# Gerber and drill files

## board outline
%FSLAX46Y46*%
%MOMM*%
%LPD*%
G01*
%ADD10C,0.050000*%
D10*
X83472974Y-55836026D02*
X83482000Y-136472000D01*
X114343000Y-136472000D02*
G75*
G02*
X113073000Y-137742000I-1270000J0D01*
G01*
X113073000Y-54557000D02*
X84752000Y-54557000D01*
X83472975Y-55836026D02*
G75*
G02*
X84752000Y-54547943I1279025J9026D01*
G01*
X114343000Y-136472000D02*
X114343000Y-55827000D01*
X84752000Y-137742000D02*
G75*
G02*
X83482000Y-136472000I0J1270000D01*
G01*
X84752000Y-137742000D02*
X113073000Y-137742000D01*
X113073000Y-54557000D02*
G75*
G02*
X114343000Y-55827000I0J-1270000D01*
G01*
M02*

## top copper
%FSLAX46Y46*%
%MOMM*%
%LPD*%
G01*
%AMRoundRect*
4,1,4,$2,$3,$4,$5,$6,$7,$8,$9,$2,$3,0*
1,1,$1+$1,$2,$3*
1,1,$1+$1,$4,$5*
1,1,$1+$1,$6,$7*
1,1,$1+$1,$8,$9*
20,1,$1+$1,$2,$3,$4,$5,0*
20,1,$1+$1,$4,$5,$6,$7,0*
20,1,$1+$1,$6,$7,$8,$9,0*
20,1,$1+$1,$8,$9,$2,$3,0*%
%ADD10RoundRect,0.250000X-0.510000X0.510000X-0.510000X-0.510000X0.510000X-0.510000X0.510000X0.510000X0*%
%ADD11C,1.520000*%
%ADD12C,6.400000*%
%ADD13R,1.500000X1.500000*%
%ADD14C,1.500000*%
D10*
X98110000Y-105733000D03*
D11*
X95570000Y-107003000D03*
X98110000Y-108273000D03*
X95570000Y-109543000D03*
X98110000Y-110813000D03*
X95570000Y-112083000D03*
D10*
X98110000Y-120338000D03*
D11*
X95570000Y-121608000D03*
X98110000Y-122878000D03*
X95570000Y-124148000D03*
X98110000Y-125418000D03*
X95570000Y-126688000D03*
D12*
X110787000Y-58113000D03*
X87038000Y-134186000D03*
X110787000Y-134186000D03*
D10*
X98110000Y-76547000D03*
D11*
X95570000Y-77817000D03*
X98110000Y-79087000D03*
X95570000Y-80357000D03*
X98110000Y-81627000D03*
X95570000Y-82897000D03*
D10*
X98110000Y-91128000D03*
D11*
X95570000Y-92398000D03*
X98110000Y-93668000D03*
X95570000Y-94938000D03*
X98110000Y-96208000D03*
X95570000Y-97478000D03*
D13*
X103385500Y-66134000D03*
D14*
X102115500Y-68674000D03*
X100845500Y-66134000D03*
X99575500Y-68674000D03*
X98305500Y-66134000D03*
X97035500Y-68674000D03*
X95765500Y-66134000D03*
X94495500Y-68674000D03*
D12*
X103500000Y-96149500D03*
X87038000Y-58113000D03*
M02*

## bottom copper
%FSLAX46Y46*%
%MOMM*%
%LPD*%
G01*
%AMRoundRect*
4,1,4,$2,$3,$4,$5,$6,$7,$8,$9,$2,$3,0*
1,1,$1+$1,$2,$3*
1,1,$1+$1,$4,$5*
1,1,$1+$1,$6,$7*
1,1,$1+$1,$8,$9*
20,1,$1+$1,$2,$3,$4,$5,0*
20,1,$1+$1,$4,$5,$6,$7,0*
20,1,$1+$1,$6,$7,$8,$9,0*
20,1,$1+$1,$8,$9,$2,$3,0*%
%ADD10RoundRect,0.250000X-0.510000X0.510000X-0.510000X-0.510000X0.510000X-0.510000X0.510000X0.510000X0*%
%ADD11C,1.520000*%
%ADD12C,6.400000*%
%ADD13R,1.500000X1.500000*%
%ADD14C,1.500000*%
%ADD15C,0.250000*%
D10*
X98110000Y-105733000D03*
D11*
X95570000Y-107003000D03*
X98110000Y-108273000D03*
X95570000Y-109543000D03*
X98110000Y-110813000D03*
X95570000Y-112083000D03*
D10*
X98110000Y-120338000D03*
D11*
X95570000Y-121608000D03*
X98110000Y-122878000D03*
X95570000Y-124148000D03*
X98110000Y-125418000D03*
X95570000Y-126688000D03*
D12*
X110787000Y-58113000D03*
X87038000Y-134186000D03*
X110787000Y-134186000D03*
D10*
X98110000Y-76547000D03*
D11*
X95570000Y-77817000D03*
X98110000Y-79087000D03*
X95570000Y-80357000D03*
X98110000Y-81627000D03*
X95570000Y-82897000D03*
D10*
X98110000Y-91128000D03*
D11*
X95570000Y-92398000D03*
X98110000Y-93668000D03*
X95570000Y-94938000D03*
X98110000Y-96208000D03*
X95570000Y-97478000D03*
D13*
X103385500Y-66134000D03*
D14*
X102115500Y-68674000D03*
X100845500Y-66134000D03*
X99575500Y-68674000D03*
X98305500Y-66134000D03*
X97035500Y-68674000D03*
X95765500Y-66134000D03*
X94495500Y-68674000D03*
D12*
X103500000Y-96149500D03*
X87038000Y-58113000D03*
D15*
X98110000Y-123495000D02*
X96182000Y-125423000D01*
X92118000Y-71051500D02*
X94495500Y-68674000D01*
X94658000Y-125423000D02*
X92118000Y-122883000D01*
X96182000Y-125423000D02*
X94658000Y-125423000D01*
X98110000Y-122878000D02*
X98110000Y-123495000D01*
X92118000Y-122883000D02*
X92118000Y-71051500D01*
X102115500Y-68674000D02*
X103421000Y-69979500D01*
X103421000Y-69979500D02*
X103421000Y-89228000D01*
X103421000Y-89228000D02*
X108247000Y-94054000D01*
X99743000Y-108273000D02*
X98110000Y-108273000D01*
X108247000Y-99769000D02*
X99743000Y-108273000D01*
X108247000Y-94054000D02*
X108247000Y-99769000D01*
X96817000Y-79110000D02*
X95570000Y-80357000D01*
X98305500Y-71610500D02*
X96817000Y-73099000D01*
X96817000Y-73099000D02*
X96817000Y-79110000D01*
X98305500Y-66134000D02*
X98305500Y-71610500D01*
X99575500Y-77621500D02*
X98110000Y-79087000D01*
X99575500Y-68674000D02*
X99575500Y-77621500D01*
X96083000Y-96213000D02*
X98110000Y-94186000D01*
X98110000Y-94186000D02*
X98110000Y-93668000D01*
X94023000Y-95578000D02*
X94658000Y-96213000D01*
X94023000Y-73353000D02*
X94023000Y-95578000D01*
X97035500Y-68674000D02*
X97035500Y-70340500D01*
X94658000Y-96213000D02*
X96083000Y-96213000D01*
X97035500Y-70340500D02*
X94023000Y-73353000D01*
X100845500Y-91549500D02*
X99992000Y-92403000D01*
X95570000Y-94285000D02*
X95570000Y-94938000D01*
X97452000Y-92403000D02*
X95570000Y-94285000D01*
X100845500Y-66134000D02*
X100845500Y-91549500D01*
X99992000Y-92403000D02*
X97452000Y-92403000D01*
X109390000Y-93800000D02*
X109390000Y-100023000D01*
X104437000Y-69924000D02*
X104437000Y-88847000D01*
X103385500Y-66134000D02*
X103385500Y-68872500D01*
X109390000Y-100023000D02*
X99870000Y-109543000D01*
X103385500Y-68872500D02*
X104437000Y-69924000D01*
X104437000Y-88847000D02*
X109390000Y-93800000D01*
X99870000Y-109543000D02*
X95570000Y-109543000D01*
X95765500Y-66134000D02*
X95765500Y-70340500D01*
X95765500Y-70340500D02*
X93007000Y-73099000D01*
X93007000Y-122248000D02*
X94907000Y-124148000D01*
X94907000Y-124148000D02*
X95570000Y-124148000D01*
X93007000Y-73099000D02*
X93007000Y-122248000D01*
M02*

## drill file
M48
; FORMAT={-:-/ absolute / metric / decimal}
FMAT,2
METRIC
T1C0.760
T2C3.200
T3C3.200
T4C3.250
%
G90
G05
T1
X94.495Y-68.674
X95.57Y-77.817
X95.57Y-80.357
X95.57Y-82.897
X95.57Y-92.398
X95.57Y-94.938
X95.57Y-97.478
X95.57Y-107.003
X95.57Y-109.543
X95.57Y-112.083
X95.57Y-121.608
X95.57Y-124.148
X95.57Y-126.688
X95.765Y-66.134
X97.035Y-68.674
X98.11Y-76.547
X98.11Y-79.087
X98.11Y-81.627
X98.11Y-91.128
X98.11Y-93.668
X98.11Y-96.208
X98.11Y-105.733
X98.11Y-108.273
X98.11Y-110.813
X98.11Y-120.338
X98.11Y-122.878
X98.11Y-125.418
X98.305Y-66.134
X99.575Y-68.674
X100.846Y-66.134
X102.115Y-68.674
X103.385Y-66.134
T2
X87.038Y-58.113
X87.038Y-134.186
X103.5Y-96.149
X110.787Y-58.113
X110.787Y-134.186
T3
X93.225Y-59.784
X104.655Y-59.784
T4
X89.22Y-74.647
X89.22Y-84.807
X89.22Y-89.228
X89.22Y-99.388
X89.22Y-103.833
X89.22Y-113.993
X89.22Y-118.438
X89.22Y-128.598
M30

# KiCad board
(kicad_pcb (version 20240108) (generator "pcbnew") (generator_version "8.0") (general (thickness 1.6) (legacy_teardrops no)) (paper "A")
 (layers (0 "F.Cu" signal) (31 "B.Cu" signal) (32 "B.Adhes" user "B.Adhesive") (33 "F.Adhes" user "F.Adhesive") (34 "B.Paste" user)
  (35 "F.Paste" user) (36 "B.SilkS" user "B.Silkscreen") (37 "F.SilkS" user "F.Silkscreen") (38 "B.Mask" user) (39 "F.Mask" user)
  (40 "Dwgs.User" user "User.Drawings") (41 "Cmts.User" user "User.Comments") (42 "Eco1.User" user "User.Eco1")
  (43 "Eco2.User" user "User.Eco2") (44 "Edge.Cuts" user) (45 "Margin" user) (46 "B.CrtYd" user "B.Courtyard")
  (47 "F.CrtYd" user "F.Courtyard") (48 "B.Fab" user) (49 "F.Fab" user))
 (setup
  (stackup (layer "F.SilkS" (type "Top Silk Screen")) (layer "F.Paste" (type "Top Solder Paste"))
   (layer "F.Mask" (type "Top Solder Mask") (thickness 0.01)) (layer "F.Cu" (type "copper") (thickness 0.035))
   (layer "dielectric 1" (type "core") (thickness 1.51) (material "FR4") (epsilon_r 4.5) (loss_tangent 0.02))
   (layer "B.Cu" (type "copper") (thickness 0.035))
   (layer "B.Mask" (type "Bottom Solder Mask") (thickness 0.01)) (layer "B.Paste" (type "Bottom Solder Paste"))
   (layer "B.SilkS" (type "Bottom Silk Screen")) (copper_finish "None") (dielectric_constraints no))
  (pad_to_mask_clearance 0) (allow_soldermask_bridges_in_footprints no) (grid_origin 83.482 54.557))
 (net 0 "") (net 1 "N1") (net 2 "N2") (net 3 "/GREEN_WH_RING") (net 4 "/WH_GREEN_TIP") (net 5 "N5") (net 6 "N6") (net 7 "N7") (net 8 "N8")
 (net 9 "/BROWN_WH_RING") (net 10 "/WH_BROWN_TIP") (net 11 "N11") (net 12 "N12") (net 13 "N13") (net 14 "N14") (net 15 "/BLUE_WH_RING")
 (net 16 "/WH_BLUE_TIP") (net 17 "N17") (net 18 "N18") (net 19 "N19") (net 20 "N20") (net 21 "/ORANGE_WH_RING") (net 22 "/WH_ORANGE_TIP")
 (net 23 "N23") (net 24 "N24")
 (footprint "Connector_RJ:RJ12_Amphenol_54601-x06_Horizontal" (layer "F.Cu") (at 98.11 105.733 -90)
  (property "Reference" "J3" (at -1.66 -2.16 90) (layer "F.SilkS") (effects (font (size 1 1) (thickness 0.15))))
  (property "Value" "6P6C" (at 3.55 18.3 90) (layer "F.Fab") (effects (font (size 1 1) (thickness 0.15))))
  (pad "" np_thru_hole circle (at -1.9 8.89 270) (size 3.25 3.25) (drill 3.25) (layers "*.Cu" "*.Mask"))
  (pad "" np_thru_hole circle (at 8.26 8.89 270) (size 3.25 3.25) (drill 3.25) (layers "*.Cu" "*.Mask"))
  (pad "1" thru_hole roundrect (at 0 0 270) (size 1.52 1.52) (drill 0.76) (layers "*.Cu" "*.Mask") (remove_unused_layers no)
   (roundrect_rratio 0.1644736842) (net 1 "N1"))
  (pad "2" thru_hole circle (at 1.27 2.54 270) (size 1.52 1.52) (drill 0.76) (layers "*.Cu" "*.Mask") (remove_unused_layers no) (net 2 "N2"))
  (pad "3" thru_hole circle (at 2.54 0 270) (size 1.52 1.52) (drill 0.76) (layers "*.Cu" "*.Mask") (remove_unused_layers no)
   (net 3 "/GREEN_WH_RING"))
  (pad "4" thru_hole circle (at 3.81 2.54 270) (size 1.52 1.52) (drill 0.76) (layers "*.Cu" "*.Mask") (remove_unused_layers no)
   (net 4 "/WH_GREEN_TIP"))
  (pad "5" thru_hole circle (at 5.08 0 270) (size 1.52 1.52) (drill 0.76) (layers "*.Cu" "*.Mask") (remove_unused_layers no) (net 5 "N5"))
  (pad "6" thru_hole circle (at 6.35 2.54 270) (size 1.52 1.52) (drill 0.76) (layers "*.Cu" "*.Mask") (remove_unused_layers no) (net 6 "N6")))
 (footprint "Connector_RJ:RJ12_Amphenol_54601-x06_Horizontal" (layer "F.Cu") (at 98.11 120.338 -90)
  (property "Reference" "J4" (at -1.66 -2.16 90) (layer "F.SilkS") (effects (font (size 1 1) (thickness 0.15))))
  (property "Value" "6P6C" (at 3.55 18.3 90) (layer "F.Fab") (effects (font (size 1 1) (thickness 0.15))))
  (pad "" np_thru_hole circle (at -1.9 8.89 270) (size 3.25 3.25) (drill 3.25) (layers "*.Cu" "*.Mask"))
  (pad "" np_thru_hole circle (at 8.26 8.89 270) (size 3.25 3.25) (drill 3.25) (layers "*.Cu" "*.Mask"))
  (pad "1" thru_hole roundrect (at 0 0 270) (size 1.52 1.52) (drill 0.76) (layers "*.Cu" "*.Mask") (remove_unused_layers no)
   (roundrect_rratio 0.1644736842) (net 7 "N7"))
  (pad "2" thru_hole circle (at 1.27 2.54 270) (size 1.52 1.52) (drill 0.76) (layers "*.Cu" "*.Mask") (remove_unused_layers no) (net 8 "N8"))
  (pad "3" thru_hole circle (at 2.54 0 270) (size 1.52 1.52) (drill 0.76) (layers "*.Cu" "*.Mask") (remove_unused_layers no)
   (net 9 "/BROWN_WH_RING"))
  (pad "4" thru_hole circle (at 3.81 2.54 270) (size 1.52 1.52) (drill 0.76) (layers "*.Cu" "*.Mask") (remove_unused_layers no)
   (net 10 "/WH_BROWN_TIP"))
  (pad "5" thru_hole circle (at 5.08 0 270) (size 1.52 1.52) (drill 0.76) (layers "*.Cu" "*.Mask") (remove_unused_layers no) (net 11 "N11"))
  (pad "6" thru_hole circle (at 6.35 2.54 270) (size 1.52 1.52) (drill 0.76) (layers "*.Cu" "*.Mask") (remove_unused_layers no)
   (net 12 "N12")))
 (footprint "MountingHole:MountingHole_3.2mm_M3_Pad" (layer "F.Cu") (at 110.787 58.113)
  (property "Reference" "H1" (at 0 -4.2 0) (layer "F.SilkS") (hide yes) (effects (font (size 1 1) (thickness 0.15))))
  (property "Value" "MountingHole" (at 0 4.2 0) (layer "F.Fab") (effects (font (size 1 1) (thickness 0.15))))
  (pad "1" thru_hole circle (at 0 0) (size 6.4 6.4) (drill 3.2) (layers "*.Cu" "*.Mask") (remove_unused_layers no)))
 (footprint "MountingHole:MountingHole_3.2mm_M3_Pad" (layer "F.Cu") (at 87.038 134.186)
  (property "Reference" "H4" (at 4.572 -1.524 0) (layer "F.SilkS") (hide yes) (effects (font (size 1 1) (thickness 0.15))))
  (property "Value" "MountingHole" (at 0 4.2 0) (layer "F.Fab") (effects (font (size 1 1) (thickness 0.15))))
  (pad "1" thru_hole circle (at 0 0) (size 6.4 6.4) (drill 3.2) (layers "*.Cu" "*.Mask") (remove_unused_layers no)))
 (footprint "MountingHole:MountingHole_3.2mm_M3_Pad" (layer "F.Cu") (at 110.787 134.186)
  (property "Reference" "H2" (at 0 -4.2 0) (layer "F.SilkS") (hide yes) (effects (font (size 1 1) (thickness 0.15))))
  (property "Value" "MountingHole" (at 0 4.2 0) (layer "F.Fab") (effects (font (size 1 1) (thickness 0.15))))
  (pad "1" thru_hole circle (at 0 0) (size 6.4 6.4) (drill 3.2) (layers "*.Cu" "*.Mask") (remove_unused_layers no)))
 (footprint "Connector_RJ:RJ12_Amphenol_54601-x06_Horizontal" (layer "F.Cu") (at 98.11 76.547 -90)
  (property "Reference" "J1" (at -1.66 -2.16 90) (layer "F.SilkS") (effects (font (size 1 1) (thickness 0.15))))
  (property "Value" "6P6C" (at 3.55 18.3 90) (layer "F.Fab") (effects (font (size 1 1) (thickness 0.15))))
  (pad "" np_thru_hole circle (at -1.9 8.89 270) (size 3.25 3.25) (drill 3.25) (layers "*.Cu" "*.Mask"))
  (pad "" np_thru_hole circle (at 8.26 8.89 270) (size 3.25 3.25) (drill 3.25) (layers "*.Cu" "*.Mask"))
  (pad "1" thru_hole roundrect (at 0 0 270) (size 1.52 1.52) (drill 0.76) (layers "*.Cu" "*.Mask") (remove_unused_layers no)
   (roundrect_rratio 0.1644736842) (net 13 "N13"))
  (pad "2" thru_hole circle (at 1.27 2.54 270) (size 1.52 1.52) (drill 0.76) (layers "*.Cu" "*.Mask") (remove_unused_layers no)
   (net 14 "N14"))
  (pad "3" thru_hole circle (at 2.54 0 270) (size 1.52 1.52) (drill 0.76) (layers "*.Cu" "*.Mask") (remove_unused_layers no)
   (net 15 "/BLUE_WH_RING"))
  (pad "4" thru_hole circle (at 3.81 2.54 270) (size 1.52 1.52) (drill 0.76) (layers "*.Cu" "*.Mask") (remove_unused_layers no)
   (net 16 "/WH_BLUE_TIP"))
  (pad "5" thru_hole circle (at 5.08 0 270) (size 1.52 1.52) (drill 0.76) (layers "*.Cu" "*.Mask") (remove_unused_layers no) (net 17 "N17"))
  (pad "6" thru_hole circle (at 6.35 2.54 270) (size 1.52 1.52) (drill 0.76) (layers "*.Cu" "*.Mask") (remove_unused_layers no)
   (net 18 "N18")))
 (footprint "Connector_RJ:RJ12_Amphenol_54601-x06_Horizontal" (layer "F.Cu") (at 98.11 91.128 -90)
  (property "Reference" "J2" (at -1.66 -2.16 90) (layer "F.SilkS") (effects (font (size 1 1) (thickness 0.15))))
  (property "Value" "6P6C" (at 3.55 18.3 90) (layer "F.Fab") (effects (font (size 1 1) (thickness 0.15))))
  (pad "" np_thru_hole circle (at -1.9 8.89 270) (size 3.25 3.25) (drill 3.25) (layers "*.Cu" "*.Mask"))
  (pad "" np_thru_hole circle (at 8.26 8.89 270) (size 3.25 3.25) (drill 3.25) (layers "*.Cu" "*.Mask"))
  (pad "1" thru_hole roundrect (at 0 0 270) (size 1.52 1.52) (drill 0.76) (layers "*.Cu" "*.Mask") (remove_unused_layers no)
   (roundrect_rratio 0.1644736842) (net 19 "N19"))
  (pad "2" thru_hole circle (at 1.27 2.54 270) (size 1.52 1.52) (drill 0.76) (layers "*.Cu" "*.Mask") (remove_unused_layers no)
   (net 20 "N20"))
  (pad "3" thru_hole circle (at 2.54 0 270) (size 1.52 1.52) (drill 0.76) (layers "*.Cu" "*.Mask") (remove_unused_layers no)
   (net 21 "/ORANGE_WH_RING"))
  (pad "4" thru_hole circle (at 3.81 2.54 270) (size 1.52 1.52) (drill 0.76) (layers "*.Cu" "*.Mask") (remove_unused_layers no)
   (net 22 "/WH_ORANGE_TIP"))
  (pad "5" thru_hole circle (at 5.08 0 270) (size 1.52 1.52) (drill 0.76) (layers "*.Cu" "*.Mask") (remove_unused_layers no) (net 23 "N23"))
  (pad "6" thru_hole circle (at 6.35 2.54 270) (size 1.52 1.52) (drill 0.76) (layers "*.Cu" "*.Mask") (remove_unused_layers no)
   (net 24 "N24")))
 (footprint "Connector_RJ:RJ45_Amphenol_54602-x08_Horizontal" (layer "F.Cu") (at 103.3855 66.134 180)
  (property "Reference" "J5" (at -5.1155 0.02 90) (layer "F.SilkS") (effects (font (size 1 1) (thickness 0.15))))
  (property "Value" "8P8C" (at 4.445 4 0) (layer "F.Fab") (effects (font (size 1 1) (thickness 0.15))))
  (pad "" np_thru_hole circle (at -1.27 6.35 180) (size 3.2 3.2) (drill 3.2) (layers "*.Cu" "*.Mask"))
  (pad "" np_thru_hole circle (at 10.16 6.35 180) (size 3.2 3.2) (drill 3.2) (layers "*.Cu" "*.Mask"))
  (pad "1" thru_hole rect (at 0 0 180) (size 1.5 1.5) (drill 0.76) (layers "*.Cu" "*.Mask") (remove_unused_layers no)
   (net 4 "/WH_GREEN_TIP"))
  (pad "2" thru_hole circle (at 1.27 -2.54 180) (size 1.5 1.5) (drill 0.76) (layers "*.Cu" "*.Mask") (remove_unused_layers no)
   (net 3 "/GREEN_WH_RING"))
  (pad "3" thru_hole circle (at 2.54 0 180) (size 1.5 1.5) (drill 0.76) (layers "*.Cu" "*.Mask") (remove_unused_layers no)
   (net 22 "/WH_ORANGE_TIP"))
  (pad "4" thru_hole circle (at 3.81 -2.54 180) (size 1.5 1.5) (drill 0.76) (layers "*.Cu" "*.Mask") (remove_unused_layers no)
   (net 15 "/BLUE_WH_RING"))
  (pad "5" thru_hole circle (at 5.08 0 180) (size 1.5 1.5) (drill 0.76) (layers "*.Cu" "*.Mask") (remove_unused_layers no)
   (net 16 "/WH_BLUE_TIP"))
  (pad "6" thru_hole circle (at 6.35 -2.54 180) (size 1.5 1.5) (drill 0.76) (layers "*.Cu" "*.Mask") (remove_unused_layers no)
   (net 21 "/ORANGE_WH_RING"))
  (pad "7" thru_hole circle (at 7.62 0 180) (size 1.5 1.5) (drill 0.76) (layers "*.Cu" "*.Mask") (remove_unused_layers no)
   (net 10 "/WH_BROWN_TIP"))
  (pad "8" thru_hole circle (at 8.89 -2.54 180) (size 1.5 1.5) (drill 0.76) (layers "*.Cu" "*.Mask") (remove_unused_layers no)
   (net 9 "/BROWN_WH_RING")))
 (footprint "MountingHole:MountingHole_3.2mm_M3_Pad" (layer "F.Cu") (at 103.5 96.1495)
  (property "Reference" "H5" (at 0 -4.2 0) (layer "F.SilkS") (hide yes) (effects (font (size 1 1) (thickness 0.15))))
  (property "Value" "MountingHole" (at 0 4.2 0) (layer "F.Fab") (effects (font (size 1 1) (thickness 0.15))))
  (pad "1" thru_hole circle (at 0 0) (size 6.4 6.4) (drill 3.2) (layers "*.Cu" "*.Mask") (remove_unused_layers no)))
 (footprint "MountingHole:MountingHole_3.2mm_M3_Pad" (layer "F.Cu") (at 87.038 58.113)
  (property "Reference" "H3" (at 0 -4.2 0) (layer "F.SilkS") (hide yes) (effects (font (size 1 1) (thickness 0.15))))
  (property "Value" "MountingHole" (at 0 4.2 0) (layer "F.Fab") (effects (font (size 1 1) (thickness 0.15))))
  (pad "1" thru_hole circle (at 0 0) (size 6.4 6.4) (drill 3.2) (layers "*.Cu" "*.Mask") (remove_unused_layers no)))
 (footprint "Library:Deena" (layer "F.Cu") (at 106.977 119.073)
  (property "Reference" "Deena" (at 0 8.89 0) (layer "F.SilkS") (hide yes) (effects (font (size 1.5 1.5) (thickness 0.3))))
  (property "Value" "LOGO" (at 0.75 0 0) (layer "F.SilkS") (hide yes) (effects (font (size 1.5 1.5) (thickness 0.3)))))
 (gr_line (start 83.472974 55.836026) (end 83.482 136.472) (stroke (width 0.05) (type default)) (layer "Edge.Cuts"))
 (gr_arc (start 114.343 136.472) (mid 113.971026 137.370026) (end 113.073 137.742) (stroke (width 0.05) (type default)) (layer "Edge.Cuts"))
 (gr_line (start 113.073 54.557) (end 84.752 54.557) (stroke (width 0.05) (type default)) (layer "Edge.Cuts"))
 (gr_arc (start 83.472975 55.836026) (mid 83.844385 54.925767) (end 84.752 54.547943) (stroke (width 0.05) (type default))
  (layer "Edge.Cuts"))
 (gr_line (start 114.343 136.472) (end 114.343 55.827) (stroke (width 0.05) (type default)) (layer "Edge.Cuts"))
 (gr_arc (start 84.752 137.742) (mid 83.853974 137.370026) (end 83.482 136.472) (stroke (width 0.05) (type default)) (layer "Edge.Cuts"))
 (gr_line (start 84.752 137.742) (end 113.073 137.742) (stroke (width 0.05) (type default)) (layer "Edge.Cuts"))
 (gr_arc (start 113.073 54.557) (mid 113.971026 54.928974) (end 114.343 55.827) (stroke (width 0.05) (type default)) (layer "Edge.Cuts"))
 (segment (start 98.11 123.495) (end 96.182 125.423) (width 0.25) (layer "B.Cu") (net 9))
 (segment (start 92.118 71.0515) (end 94.4955 68.674) (width 0.25) (layer "B.Cu") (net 9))
 (segment (start 94.658 125.423) (end 92.118 122.883) (width 0.25) (layer "B.Cu") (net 9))
 (segment (start 96.182 125.423) (end 94.658 125.423) (width 0.25) (layer "B.Cu") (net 9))
 (segment (start 98.11 122.878) (end 98.11 123.495) (width 0.25) (layer "B.Cu") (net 9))
 (segment (start 92.118 122.883) (end 92.118 71.0515) (width 0.25) (layer "B.Cu") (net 9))
 (segment (start 102.1155 68.674) (end 103.421 69.9795) (width 0.25) (layer "B.Cu") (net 3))
 (segment (start 103.421 69.9795) (end 103.421 89.228) (width 0.25) (layer "B.Cu") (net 3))
 (segment (start 103.421 89.228) (end 108.247 94.054) (width 0.25) (layer "B.Cu") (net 3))
 (segment (start 99.743 108.273) (end 98.11 108.273) (width 0.25) (layer "B.Cu") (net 3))
 (segment (start 108.247 99.769) (end 99.743 108.273) (width 0.25) (layer "B.Cu") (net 3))
 (segment (start 108.247 94.054) (end 108.247 99.769) (width 0.25) (layer "B.Cu") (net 3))
 (segment (start 96.817 79.11) (end 95.57 80.357) (width 0.25) (layer "B.Cu") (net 16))
 (segment (start 98.3055 71.6105) (end 96.817 73.099) (width 0.25) (layer "B.Cu") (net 16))
 (segment (start 96.817 73.099) (end 96.817 79.11) (width 0.25) (layer "B.Cu") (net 16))
 (segment (start 98.3055 66.134) (end 98.3055 71.6105) (width 0.25) (layer "B.Cu") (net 16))
 (segment (start 99.5755 77.6215) (end 98.11 79.087) (width 0.25) (layer "B.Cu") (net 15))
 (segment (start 99.5755 68.674) (end 99.5755 77.6215) (width 0.25) (layer "B.Cu") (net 15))
 (segment (start 96.083 96.213) (end 98.11 94.186) (width 0.25) (layer "B.Cu") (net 21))
 (segment (start 98.11 94.186) (end 98.11 93.668) (width 0.25) (layer "B.Cu") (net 21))
 (segment (start 94.023 95.578) (end 94.658 96.213) (width 0.25) (layer "B.Cu") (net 21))
 (segment (start 94.023 73.353) (end 94.023 95.578) (width 0.25) (layer "B.Cu") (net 21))
 (segment (start 97.0355 68.674) (end 97.0355 70.3405) (width 0.25) (layer "B.Cu") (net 21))
 (segment (start 94.658 96.213) (end 96.083 96.213) (width 0.25) (layer "B.Cu") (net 21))
 (segment (start 97.0355 70.3405) (end 94.023 73.353) (width 0.25) (layer "B.Cu") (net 21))
 (segment (start 100.8455 91.5495) (end 99.992 92.403) (width 0.25) (layer "B.Cu") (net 22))
 (segment (start 95.57 94.285) (end 95.57 94.938) (width 0.25) (layer "B.Cu") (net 22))
 (segment (start 97.452 92.403) (end 95.57 94.285) (width 0.25) (layer "B.Cu") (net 22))
 (segment (start 100.8455 66.134) (end 100.8455 91.5495) (width 0.25) (layer "B.Cu") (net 22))
 (segment (start 99.992 92.403) (end 97.452 92.403) (width 0.25) (layer "B.Cu") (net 22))
 (segment (start 109.39 93.8) (end 109.39 100.023) (width 0.25) (layer "B.Cu") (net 4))
 (segment (start 104.437 69.924) (end 104.437 88.847) (width 0.25) (layer "B.Cu") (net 4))
 (segment (start 103.3855 66.134) (end 103.3855 68.8725) (width 0.25) (layer "B.Cu") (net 4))
 (segment (start 109.39 100.023) (end 99.87 109.543) (width 0.25) (layer "B.Cu") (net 4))
 (segment (start 103.3855 68.8725) (end 104.437 69.924) (width 0.25) (layer "B.Cu") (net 4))
 (segment (start 104.437 88.847) (end 109.39 93.8) (width 0.25) (layer "B.Cu") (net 4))
 (segment (start 99.87 109.543) (end 95.57 109.543) (width 0.25) (layer "B.Cu") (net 4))
 (segment (start 95.7655 66.134) (end 95.7655 70.3405) (width 0.25) (layer "B.Cu") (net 10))
 (segment (start 95.7655 70.3405) (end 93.007 73.099) (width 0.25) (layer "B.Cu") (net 10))
 (segment (start 93.007 122.248) (end 94.907 124.148) (width 0.25) (layer "B.Cu") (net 10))
 (segment (start 94.907 124.148) (end 95.57 124.148) (width 0.25) (layer "B.Cu") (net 10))
 (segment (start 93.007 73.099) (end 93.007 122.248) (width 0.25) (layer "B.Cu") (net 10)))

